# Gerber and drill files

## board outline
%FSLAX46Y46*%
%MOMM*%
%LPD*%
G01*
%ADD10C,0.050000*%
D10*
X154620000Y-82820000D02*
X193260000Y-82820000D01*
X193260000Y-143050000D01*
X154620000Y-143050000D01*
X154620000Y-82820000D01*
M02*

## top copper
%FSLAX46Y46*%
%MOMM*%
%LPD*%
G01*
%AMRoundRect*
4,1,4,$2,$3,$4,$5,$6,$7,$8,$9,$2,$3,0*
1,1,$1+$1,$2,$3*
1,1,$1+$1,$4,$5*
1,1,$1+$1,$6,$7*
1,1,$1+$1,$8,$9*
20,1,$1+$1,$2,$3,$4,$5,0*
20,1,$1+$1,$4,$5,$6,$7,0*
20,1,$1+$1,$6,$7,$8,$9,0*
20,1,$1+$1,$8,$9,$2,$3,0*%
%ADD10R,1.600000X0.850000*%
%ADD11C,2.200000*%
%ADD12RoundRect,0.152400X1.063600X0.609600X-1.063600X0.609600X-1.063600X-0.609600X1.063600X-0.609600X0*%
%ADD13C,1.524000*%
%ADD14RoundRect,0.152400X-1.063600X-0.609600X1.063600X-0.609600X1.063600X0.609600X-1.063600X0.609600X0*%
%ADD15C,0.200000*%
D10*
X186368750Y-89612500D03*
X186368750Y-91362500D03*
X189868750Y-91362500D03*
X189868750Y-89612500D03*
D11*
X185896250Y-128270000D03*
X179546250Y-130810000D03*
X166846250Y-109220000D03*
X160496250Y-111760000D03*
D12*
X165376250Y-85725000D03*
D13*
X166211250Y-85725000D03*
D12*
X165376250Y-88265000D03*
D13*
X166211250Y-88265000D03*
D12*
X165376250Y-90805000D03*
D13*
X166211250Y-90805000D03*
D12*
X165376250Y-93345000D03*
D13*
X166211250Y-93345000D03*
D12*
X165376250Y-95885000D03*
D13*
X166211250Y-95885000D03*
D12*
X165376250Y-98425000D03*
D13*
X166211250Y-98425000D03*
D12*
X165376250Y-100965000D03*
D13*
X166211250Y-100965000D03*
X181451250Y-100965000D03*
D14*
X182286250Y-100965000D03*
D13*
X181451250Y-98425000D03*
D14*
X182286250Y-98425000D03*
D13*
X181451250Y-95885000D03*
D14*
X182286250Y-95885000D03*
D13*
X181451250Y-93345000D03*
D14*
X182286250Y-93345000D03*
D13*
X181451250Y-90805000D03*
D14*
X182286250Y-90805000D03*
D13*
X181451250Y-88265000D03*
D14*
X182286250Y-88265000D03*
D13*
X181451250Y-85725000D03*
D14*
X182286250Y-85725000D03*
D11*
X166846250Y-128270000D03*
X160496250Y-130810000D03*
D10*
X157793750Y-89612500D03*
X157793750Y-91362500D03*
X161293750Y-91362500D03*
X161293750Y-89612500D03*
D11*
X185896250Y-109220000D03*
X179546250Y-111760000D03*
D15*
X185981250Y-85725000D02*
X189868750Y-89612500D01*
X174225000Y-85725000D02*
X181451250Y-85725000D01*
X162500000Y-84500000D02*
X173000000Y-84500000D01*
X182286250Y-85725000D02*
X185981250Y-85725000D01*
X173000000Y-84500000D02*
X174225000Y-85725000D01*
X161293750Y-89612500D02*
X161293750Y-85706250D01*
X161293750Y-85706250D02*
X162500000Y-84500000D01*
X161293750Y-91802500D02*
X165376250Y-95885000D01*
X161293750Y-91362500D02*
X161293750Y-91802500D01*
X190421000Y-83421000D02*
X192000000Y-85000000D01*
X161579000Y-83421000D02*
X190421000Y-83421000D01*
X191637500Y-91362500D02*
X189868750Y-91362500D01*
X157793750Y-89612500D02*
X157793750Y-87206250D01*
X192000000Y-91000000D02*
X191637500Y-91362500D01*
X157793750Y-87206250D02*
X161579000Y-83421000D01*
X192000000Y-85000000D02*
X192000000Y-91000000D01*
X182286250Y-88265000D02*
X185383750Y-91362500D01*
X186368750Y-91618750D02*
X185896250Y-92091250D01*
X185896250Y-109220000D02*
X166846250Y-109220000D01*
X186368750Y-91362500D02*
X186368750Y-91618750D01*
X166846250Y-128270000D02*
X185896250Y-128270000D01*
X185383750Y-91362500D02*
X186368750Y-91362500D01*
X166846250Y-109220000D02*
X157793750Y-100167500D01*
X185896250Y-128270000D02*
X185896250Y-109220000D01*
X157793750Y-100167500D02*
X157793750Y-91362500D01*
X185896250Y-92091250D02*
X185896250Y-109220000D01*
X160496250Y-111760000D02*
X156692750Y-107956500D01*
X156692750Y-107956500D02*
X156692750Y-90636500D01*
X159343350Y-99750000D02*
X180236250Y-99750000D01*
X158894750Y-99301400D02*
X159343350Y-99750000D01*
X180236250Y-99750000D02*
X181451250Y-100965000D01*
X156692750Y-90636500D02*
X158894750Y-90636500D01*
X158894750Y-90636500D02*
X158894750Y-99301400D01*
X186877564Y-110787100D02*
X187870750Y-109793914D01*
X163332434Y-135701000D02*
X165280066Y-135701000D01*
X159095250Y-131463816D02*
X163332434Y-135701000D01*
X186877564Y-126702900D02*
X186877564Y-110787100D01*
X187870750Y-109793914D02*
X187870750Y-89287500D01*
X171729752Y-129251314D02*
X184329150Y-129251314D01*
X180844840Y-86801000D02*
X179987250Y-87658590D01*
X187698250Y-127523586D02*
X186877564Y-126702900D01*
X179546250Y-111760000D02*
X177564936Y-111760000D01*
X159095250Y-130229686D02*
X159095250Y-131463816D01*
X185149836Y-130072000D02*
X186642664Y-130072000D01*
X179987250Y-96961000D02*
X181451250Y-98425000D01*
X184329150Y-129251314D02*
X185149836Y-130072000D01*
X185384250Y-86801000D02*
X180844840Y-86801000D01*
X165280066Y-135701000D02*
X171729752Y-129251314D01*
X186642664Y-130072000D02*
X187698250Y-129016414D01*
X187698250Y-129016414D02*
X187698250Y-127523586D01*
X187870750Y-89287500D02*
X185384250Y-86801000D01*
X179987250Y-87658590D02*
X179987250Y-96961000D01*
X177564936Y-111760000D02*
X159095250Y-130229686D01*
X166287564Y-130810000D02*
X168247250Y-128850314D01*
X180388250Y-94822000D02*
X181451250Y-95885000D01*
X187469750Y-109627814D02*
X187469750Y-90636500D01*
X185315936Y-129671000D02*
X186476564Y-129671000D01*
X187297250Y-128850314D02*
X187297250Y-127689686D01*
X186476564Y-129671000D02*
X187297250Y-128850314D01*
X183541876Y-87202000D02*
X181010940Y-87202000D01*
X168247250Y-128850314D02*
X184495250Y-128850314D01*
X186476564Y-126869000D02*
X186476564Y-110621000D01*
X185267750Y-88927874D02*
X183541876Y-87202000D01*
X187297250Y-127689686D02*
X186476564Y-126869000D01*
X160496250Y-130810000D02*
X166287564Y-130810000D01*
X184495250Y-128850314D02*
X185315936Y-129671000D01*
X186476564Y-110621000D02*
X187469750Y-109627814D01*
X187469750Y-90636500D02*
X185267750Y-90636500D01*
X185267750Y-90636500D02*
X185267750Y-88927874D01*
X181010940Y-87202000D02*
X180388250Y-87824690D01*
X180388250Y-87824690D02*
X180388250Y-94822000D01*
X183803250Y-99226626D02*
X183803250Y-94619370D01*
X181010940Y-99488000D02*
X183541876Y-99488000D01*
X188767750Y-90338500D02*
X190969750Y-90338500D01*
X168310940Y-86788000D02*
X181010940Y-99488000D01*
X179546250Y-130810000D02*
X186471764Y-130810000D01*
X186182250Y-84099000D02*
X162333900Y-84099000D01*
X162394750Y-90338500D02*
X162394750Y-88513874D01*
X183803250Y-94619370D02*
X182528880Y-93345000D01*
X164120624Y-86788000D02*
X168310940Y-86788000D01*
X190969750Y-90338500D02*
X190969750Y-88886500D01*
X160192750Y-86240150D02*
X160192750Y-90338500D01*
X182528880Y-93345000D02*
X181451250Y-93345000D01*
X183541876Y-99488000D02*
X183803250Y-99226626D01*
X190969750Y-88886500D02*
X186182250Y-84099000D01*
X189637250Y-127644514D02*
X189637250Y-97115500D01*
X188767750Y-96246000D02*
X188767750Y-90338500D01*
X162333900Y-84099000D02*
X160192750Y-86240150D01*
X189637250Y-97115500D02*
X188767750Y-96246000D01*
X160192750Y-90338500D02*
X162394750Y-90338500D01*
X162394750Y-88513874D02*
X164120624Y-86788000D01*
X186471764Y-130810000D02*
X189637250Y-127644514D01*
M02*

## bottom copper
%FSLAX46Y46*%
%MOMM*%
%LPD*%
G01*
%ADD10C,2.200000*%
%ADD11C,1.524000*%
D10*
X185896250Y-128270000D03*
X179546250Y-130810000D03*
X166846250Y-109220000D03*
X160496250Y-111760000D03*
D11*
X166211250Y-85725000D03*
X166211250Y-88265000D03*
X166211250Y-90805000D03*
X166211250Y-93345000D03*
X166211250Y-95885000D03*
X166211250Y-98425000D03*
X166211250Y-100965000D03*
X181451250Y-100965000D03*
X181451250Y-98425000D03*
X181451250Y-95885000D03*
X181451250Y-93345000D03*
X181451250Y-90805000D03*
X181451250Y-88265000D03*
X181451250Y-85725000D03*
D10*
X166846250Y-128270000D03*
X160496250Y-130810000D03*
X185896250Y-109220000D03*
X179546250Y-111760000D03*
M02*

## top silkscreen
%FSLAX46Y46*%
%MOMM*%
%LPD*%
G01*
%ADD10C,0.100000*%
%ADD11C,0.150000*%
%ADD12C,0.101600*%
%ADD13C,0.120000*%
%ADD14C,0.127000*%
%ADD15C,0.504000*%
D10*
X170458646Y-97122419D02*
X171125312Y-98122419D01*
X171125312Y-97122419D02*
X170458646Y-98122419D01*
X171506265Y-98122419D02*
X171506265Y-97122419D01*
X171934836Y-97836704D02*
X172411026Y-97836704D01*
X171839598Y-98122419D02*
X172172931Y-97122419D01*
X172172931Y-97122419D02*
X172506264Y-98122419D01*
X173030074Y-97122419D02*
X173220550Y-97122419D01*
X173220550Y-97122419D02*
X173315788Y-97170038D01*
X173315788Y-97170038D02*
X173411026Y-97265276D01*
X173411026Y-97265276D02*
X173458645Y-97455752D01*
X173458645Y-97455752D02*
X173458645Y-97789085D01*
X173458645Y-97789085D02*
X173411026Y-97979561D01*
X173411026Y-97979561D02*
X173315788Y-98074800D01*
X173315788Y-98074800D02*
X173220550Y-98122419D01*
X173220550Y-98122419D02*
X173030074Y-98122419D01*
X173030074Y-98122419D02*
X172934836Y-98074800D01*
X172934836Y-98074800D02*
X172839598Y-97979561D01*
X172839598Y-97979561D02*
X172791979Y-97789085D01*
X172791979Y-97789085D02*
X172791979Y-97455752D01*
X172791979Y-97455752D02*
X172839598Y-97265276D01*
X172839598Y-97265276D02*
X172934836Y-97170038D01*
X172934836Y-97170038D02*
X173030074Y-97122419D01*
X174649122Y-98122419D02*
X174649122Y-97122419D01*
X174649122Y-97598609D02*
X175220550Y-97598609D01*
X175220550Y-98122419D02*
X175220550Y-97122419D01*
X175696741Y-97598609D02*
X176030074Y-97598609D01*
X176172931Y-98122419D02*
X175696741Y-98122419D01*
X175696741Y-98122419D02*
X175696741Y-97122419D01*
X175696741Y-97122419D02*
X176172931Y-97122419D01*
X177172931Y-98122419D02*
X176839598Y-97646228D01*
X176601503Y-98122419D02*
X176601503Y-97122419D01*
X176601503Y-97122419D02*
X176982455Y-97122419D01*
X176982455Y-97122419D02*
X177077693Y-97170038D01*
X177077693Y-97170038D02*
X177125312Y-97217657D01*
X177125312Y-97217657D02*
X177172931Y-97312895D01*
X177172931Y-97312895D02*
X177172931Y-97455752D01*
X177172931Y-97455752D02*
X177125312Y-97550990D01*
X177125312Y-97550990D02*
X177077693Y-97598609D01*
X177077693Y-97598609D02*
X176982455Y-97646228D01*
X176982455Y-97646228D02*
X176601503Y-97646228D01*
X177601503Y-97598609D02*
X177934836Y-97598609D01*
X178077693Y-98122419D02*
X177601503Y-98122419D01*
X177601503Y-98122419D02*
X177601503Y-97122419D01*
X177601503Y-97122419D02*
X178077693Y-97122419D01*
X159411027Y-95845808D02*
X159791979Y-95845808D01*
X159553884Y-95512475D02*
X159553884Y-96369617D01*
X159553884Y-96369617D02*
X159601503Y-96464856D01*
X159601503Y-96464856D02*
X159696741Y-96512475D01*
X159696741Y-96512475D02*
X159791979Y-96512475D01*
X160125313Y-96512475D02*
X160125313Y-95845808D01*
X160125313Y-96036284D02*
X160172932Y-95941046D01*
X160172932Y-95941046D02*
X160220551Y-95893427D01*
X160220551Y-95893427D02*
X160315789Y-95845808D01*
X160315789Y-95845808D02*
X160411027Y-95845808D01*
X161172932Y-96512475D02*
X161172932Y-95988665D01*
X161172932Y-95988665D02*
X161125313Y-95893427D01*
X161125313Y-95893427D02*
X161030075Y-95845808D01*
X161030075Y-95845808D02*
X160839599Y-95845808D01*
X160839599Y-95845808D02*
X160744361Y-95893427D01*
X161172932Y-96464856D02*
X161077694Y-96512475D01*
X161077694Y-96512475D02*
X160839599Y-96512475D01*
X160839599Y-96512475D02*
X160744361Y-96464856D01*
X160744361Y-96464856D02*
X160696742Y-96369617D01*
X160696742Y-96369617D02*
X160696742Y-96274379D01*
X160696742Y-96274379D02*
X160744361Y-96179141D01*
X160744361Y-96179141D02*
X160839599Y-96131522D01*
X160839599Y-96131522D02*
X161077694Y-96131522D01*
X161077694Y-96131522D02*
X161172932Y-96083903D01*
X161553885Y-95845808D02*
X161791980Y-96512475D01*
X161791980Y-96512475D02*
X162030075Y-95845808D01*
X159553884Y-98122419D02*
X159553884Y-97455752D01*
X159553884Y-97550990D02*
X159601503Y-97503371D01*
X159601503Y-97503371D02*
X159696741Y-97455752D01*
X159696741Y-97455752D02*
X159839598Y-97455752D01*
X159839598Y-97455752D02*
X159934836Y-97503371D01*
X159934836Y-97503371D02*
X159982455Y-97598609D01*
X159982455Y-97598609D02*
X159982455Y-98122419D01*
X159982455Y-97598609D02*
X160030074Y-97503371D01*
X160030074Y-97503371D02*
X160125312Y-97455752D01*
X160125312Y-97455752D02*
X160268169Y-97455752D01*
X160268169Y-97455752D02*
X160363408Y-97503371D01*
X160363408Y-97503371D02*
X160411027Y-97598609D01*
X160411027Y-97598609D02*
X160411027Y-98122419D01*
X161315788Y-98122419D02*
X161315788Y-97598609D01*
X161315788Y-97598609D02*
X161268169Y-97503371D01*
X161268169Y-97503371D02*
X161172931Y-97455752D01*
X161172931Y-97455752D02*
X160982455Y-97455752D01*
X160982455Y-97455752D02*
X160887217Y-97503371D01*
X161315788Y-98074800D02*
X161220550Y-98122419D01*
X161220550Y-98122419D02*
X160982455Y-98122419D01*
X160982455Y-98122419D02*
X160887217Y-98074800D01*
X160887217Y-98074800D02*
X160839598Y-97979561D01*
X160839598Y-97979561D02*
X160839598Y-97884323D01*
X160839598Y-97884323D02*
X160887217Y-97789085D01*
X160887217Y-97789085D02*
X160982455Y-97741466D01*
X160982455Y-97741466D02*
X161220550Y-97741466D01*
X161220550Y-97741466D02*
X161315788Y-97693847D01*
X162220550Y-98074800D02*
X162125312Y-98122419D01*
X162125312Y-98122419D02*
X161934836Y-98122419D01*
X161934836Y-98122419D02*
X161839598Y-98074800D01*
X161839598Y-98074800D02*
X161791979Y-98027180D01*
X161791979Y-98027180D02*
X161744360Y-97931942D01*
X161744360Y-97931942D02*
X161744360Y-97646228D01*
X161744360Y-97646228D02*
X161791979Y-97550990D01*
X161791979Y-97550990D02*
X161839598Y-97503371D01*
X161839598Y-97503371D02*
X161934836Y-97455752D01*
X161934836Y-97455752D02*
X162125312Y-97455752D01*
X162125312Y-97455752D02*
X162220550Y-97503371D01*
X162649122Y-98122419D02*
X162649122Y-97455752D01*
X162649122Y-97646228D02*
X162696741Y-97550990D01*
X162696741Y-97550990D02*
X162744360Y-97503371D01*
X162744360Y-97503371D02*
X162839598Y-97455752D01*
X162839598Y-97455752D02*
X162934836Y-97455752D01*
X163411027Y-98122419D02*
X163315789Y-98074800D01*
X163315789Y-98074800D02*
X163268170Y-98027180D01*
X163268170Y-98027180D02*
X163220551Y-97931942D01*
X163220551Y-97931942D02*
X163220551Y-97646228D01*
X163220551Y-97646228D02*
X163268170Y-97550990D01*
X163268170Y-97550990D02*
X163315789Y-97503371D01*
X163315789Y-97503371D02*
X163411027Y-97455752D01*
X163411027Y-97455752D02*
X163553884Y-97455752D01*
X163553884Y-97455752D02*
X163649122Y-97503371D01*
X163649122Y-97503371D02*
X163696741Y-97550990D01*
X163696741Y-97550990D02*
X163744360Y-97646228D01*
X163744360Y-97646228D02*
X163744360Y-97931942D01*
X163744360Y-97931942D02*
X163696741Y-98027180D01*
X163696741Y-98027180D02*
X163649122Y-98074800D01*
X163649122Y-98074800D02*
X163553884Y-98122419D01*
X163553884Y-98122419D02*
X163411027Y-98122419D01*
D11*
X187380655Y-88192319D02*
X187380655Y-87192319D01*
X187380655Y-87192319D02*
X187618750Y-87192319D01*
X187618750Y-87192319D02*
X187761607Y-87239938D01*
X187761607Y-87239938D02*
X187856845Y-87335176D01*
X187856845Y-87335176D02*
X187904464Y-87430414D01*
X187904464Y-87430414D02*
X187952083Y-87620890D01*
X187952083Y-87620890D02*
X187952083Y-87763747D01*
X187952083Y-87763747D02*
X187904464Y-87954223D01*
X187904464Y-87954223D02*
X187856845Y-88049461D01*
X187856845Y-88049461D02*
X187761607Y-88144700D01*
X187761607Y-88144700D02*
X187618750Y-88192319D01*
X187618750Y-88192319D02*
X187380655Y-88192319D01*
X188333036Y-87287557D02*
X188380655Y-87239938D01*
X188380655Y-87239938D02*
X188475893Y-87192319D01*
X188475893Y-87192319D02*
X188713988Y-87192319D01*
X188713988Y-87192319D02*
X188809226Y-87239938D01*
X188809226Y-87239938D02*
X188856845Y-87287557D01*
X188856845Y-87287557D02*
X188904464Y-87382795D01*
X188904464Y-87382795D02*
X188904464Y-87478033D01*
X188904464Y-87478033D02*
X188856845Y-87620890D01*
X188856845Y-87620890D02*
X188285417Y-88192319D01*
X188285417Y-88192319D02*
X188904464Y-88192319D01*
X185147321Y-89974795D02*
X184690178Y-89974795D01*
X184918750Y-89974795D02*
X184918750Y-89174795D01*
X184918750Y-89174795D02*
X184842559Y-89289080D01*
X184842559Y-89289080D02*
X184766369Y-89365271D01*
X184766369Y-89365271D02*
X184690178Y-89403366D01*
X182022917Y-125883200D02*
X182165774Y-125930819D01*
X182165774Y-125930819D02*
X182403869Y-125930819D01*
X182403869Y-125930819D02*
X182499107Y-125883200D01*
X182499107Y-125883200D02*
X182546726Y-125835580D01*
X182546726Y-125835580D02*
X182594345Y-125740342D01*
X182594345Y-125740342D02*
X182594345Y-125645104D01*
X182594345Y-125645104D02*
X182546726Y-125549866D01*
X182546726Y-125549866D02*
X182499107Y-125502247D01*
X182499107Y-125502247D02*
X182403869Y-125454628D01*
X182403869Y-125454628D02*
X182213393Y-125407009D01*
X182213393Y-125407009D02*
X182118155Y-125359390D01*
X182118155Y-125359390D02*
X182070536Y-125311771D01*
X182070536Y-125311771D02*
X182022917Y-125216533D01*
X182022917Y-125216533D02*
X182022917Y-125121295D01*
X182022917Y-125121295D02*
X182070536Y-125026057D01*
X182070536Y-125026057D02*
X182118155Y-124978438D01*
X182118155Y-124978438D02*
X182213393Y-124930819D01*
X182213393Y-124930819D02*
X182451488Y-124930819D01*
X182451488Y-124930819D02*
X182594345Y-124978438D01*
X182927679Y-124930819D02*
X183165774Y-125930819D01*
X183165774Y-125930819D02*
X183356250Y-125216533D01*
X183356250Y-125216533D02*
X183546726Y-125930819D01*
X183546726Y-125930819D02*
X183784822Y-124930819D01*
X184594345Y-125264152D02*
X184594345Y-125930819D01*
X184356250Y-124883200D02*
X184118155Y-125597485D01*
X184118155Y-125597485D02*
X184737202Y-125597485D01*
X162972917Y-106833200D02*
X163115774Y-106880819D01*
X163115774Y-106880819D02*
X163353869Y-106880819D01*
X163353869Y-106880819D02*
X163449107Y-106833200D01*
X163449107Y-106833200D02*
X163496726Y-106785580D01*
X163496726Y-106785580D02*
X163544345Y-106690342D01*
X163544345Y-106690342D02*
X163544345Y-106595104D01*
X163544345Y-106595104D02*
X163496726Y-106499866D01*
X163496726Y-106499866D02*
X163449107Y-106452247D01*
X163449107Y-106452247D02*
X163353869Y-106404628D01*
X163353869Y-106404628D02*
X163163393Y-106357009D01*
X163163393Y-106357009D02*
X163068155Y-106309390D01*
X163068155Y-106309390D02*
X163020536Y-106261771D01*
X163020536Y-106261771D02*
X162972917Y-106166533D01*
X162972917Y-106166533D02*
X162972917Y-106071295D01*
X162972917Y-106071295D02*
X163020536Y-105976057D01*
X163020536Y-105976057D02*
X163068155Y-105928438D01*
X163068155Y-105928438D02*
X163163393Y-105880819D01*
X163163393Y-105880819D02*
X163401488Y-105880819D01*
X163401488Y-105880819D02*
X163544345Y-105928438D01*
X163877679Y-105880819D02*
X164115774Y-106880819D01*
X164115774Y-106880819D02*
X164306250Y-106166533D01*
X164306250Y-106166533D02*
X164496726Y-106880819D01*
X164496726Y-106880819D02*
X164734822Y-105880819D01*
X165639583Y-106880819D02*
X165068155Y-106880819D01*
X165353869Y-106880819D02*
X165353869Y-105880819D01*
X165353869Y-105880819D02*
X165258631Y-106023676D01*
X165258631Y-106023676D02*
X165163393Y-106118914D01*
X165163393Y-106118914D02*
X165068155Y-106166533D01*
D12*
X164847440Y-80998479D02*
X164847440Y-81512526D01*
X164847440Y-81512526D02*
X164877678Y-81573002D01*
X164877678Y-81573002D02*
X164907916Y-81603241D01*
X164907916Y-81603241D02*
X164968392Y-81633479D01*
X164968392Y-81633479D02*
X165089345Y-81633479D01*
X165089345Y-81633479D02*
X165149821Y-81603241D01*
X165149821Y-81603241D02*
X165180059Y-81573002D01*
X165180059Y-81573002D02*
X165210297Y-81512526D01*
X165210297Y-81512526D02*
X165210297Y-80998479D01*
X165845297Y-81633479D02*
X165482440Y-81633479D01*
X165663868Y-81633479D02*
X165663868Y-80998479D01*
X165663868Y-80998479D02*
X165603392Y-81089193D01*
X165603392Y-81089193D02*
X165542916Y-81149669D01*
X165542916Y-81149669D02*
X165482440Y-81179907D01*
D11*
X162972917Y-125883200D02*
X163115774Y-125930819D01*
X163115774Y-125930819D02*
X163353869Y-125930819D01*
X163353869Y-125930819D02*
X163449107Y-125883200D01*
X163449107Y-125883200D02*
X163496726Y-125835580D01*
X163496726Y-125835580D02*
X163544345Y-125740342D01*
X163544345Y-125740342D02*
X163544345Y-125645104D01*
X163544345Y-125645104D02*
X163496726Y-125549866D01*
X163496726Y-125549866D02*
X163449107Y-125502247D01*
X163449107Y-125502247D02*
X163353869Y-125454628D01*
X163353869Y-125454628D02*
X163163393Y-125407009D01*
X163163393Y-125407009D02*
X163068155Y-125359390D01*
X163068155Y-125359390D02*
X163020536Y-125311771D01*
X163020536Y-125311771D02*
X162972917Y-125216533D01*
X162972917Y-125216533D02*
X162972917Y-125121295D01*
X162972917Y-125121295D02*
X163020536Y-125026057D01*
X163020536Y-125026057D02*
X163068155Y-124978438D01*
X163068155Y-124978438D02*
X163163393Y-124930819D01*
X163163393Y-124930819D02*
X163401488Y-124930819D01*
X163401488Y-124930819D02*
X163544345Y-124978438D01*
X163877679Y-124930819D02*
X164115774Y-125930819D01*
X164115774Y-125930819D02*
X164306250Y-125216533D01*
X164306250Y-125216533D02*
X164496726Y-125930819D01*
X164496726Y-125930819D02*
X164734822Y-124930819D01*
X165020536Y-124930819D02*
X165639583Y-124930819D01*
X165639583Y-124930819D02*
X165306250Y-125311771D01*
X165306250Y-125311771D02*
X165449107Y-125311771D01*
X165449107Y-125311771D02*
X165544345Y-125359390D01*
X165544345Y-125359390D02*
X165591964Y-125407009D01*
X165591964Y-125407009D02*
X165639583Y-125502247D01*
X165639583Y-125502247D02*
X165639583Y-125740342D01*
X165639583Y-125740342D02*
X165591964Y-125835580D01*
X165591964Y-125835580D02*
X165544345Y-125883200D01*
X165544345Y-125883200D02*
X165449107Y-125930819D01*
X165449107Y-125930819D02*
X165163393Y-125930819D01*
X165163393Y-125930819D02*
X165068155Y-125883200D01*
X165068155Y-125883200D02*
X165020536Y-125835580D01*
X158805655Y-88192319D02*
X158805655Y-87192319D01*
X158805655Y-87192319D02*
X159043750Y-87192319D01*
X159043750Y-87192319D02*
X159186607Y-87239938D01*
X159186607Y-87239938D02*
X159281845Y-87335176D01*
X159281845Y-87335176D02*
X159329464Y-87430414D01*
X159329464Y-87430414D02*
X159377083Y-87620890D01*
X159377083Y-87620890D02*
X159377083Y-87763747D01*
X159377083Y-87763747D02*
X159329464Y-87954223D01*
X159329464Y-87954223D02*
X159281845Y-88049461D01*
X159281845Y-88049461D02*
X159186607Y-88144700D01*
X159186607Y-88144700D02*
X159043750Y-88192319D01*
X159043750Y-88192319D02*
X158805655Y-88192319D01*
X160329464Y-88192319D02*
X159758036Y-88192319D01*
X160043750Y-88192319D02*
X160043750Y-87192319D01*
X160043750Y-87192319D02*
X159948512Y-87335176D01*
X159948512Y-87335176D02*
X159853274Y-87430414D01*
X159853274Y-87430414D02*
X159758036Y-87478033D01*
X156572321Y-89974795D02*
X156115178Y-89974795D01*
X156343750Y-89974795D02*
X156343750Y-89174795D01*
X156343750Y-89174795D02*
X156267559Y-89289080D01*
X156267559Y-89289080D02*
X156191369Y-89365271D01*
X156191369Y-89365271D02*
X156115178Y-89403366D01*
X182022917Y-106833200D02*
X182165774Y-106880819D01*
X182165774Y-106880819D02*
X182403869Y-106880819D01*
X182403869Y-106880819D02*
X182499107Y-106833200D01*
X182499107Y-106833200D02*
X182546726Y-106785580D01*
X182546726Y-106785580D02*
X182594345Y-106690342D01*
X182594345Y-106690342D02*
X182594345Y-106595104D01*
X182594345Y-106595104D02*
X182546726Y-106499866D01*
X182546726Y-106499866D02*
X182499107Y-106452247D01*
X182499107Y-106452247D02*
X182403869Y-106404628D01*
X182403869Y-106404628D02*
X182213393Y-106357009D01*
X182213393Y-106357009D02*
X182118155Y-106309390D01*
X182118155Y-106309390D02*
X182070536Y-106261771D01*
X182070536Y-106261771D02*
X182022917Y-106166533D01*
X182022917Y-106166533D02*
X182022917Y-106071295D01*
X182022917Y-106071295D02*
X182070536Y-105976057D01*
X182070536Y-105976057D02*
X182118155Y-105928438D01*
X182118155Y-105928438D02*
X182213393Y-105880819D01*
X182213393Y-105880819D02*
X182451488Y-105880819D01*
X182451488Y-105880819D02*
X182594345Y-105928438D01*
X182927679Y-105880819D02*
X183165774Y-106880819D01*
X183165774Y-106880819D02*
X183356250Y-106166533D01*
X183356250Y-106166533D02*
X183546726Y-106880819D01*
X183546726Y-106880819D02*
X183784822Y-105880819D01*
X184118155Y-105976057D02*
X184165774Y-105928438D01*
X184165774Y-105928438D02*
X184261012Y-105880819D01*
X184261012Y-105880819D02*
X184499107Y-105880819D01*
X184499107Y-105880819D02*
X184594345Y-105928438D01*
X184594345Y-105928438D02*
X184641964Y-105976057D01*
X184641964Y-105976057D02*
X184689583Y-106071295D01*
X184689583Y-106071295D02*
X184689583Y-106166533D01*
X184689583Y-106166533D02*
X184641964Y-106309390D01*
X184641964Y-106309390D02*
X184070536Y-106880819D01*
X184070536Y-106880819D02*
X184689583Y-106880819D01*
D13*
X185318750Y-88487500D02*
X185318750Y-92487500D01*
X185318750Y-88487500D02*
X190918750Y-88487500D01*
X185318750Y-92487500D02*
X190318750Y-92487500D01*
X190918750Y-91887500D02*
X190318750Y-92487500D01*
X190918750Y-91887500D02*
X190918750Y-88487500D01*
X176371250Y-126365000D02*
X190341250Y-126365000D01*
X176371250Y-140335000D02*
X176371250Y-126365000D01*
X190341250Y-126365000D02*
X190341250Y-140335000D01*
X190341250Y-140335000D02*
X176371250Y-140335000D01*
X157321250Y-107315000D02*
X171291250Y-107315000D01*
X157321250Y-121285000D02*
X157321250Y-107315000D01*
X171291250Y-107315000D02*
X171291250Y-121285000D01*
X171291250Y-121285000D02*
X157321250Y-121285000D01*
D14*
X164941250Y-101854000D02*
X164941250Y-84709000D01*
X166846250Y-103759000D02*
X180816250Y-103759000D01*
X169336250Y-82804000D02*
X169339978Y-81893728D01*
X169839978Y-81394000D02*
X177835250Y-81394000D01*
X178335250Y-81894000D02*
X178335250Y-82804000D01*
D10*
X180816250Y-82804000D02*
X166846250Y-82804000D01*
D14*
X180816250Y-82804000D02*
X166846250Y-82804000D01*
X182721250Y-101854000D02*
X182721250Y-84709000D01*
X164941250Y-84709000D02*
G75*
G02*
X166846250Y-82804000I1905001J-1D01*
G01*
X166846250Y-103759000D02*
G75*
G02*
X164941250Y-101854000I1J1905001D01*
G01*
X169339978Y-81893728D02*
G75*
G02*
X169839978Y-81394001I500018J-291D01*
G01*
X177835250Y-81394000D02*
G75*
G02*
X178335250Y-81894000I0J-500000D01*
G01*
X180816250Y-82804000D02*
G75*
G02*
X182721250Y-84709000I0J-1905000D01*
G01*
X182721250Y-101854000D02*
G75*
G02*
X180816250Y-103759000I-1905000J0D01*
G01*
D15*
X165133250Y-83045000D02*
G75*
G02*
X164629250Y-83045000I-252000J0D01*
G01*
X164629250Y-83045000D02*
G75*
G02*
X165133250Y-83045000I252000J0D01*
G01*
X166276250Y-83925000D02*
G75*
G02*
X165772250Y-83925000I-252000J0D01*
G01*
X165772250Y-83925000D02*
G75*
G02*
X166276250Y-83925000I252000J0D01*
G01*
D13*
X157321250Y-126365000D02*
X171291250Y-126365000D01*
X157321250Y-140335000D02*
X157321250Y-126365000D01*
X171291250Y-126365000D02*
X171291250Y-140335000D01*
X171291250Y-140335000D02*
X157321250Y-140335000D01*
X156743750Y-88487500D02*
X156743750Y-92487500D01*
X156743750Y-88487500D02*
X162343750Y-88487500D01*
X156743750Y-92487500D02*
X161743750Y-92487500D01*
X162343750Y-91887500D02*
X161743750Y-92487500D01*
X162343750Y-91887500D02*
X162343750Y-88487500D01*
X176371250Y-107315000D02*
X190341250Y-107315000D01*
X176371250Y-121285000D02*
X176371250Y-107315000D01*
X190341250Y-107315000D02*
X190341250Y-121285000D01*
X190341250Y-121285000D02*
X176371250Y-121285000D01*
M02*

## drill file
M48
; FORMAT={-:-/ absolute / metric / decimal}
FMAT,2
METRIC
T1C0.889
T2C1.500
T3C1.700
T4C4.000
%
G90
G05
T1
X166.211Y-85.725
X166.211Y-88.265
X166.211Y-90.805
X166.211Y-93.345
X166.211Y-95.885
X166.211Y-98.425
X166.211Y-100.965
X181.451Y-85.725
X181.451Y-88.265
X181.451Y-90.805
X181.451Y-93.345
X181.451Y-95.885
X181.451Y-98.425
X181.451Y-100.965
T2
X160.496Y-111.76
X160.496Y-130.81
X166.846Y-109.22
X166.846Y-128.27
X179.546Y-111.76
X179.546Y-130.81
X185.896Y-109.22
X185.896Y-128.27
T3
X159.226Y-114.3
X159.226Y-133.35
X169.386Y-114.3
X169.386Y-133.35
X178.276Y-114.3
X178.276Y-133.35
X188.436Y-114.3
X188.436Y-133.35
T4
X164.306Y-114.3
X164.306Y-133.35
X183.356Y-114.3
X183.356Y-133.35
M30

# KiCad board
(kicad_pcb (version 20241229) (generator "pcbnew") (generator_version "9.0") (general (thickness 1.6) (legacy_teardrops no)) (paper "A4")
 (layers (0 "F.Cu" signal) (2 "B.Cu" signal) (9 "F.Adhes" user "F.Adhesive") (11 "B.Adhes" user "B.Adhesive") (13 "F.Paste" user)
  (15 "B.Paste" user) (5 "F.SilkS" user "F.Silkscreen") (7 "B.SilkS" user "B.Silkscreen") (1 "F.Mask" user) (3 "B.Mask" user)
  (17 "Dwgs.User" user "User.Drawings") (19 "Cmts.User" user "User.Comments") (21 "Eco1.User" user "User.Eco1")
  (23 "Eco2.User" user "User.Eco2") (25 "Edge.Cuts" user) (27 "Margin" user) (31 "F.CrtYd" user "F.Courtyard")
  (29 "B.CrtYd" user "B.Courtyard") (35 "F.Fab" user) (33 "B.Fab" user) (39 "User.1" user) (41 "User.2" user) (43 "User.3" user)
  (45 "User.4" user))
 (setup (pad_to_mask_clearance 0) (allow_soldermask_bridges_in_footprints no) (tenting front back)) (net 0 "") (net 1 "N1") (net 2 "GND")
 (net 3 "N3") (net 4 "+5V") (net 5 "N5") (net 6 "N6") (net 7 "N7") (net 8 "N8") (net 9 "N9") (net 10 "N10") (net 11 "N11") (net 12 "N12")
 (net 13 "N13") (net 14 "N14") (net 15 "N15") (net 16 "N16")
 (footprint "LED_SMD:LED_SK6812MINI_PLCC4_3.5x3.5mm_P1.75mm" (layer "F.Cu") (at 188.11875 90.4875)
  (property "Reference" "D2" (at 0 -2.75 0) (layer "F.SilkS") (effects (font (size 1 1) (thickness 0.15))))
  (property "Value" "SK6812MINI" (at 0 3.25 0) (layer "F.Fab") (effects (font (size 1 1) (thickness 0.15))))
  (fp_line (start -2.8 -2) (end -2.8 2) (stroke (width 0.12) (type default)) (layer "F.SilkS"))
  (fp_line (start -2.8 -2) (end 2.8 -2) (stroke (width 0.12) (type solid)) (layer "F.SilkS"))
  (fp_line (start -2.8 2) (end 2.2 2) (stroke (width 0.12) (type solid)) (layer "F.SilkS"))
  (fp_line (start 2.8 1.4) (end 2.2 2) (stroke (width 0.12) (type default)) (layer "F.SilkS"))
  (fp_line (start 2.8 1.4) (end 2.8 -2) (stroke (width 0.12) (type solid)) (layer "F.SilkS"))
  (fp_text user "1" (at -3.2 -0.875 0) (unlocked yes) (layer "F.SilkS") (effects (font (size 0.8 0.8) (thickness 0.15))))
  (pad "1" smd rect (at -1.75 -0.875) (size 1.6 0.85) (layers "F.Cu" "F.Mask" "F.Paste") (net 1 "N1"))
  (pad "2" smd rect (at -1.75 0.875) (size 1.6 0.85) (layers "F.Cu" "F.Mask" "F.Paste") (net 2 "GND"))
  (pad "3" smd rect (at 1.75 0.875) (size 1.6 0.85) (layers "F.Cu" "F.Mask" "F.Paste") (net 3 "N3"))
  (pad "4" smd rect (at 1.75 -0.875) (size 1.6 0.85) (layers "F.Cu" "F.Mask" "F.Paste") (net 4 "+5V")))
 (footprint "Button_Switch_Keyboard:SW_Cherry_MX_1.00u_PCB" (layer "F.Cu") (at 185.89625 128.27)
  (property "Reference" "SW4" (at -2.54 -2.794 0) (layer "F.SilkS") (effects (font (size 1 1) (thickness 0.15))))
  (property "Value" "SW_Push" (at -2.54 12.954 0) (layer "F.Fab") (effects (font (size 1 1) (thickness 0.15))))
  (fp_line (start -9.525 -1.905) (end 4.445 -1.905) (stroke (width 0.12) (type solid)) (layer "F.SilkS"))
  (fp_line (start -9.525 12.065) (end -9.525 -1.905) (stroke (width 0.12) (type solid)) (layer "F.SilkS"))
  (fp_line (start 4.445 -1.905) (end 4.445 12.065) (stroke (width 0.12) (type solid)) (layer "F.SilkS"))
  (fp_line (start 4.445 12.065) (end -9.525 12.065) (stroke (width 0.12) (type solid)) (layer "F.SilkS"))
  (pad "" np_thru_hole circle (at -7.62 5.08) (size 1.7 1.7) (drill 1.7) (layers "*.Cu" "*.Mask"))
  (pad "" np_thru_hole circle (at -2.54 5.08) (size 4 4) (drill 4) (layers "*.Cu" "*.Mask"))
  (pad "" np_thru_hole circle (at 2.54 5.08) (size 1.7 1.7) (drill 1.7) (layers "*.Cu" "*.Mask"))
  (pad "1" thru_hole circle (at 0 0) (size 2.2 2.2) (drill 1.5) (layers "*.Cu" "*.Mask") (remove_unused_layers no) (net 2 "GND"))
  (pad "2" thru_hole circle (at -6.35 2.54) (size 2.2 2.2) (drill 1.5) (layers "*.Cu" "*.Mask") (remove_unused_layers no) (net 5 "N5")))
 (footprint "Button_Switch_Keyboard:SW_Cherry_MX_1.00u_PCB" (layer "F.Cu") (at 166.84625 109.22)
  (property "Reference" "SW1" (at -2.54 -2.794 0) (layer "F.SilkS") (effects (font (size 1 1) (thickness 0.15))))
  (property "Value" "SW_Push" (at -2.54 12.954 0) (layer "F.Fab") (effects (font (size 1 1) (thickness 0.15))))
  (fp_line (start -9.525 -1.905) (end 4.445 -1.905) (stroke (width 0.12) (type solid)) (layer "F.SilkS"))
  (fp_line (start -9.525 12.065) (end -9.525 -1.905) (stroke (width 0.12) (type solid)) (layer "F.SilkS"))
  (fp_line (start 4.445 -1.905) (end 4.445 12.065) (stroke (width 0.12) (type solid)) (layer "F.SilkS"))
  (fp_line (start 4.445 12.065) (end -9.525 12.065) (stroke (width 0.12) (type solid)) (layer "F.SilkS"))
  (pad "" np_thru_hole circle (at -7.62 5.08) (size 1.7 1.7) (drill 1.7) (layers "*.Cu" "*.Mask"))
  (pad "" np_thru_hole circle (at -2.54 5.08) (size 4 4) (drill 4) (layers "*.Cu" "*.Mask"))
  (pad "" np_thru_hole circle (at 2.54 5.08) (size 1.7 1.7) (drill 1.7) (layers "*.Cu" "*.Mask"))
  (pad "1" thru_hole circle (at 0 0) (size 2.2 2.2) (drill 1.5) (layers "*.Cu" "*.Mask") (remove_unused_layers no) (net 2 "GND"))
  (pad "2" thru_hole circle (at -6.35 2.54) (size 2.2 2.2) (drill 1.5) (layers "*.Cu" "*.Mask") (remove_unused_layers no) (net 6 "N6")))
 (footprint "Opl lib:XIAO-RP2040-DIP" (layer "F.Cu") (at 173.83125 93.345)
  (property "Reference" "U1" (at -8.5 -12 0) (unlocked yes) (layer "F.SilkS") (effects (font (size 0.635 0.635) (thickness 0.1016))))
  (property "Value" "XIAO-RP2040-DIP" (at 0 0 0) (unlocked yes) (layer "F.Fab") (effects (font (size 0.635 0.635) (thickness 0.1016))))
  (fp_line (start -8.89 8.509) (end -8.89 -8.636) (stroke (width 0.127) (type solid)) (layer "F.SilkS"))
  (fp_line (start -6.985 10.414) (end 6.985 10.414) (stroke (width 0.127) (type solid)) (layer "F.SilkS"))
  (fp_line (start -4.495 -10.541) (end -4.491272 -11.451272) (stroke (width 0.127) (type solid)) (layer "F.SilkS"))
  (fp_line (start -3.991272 -11.951) (end 4.004 -11.951) (stroke (width 0.127) (type solid)) (layer "F.SilkS"))
  (fp_line (start 4.504 -11.451) (end 4.504 -10.541) (stroke (width 0.127) (type solid)) (layer "F.SilkS"))
  (fp_line (start 6.985 -10.541) (end -6.985 -10.541) (stroke (width 0.1) (type solid)) (layer "F.SilkS"))
  (fp_line (start 6.985 -10.541) (end -6.985 -10.541) (stroke (width 0.127) (type solid)) (layer "F.SilkS"))
  (fp_line (start 8.89 8.509) (end 8.89 -8.636) (stroke (width 0.127) (type solid)) (layer "F.SilkS"))
  (fp_arc (start -8.89 -8.636) (mid -8.332038 -9.983038) (end -6.985 -10.541) (stroke (width 0.127) (type solid)) (layer "F.SilkS"))
  (fp_arc (start -6.985 10.414) (mid -8.332038 9.856038) (end -8.89 8.509) (stroke (width 0.127) (type solid)) (layer "F.SilkS"))
  (fp_arc (start -4.491272 -11.451272) (mid -4.344728 -11.80464) (end -3.991272 -11.951) (stroke (width 0.127) (type default))
   (layer "F.SilkS"))
  (fp_arc (start 4.004 -11.951) (mid 4.357553 -11.804553) (end 4.504 -11.451) (stroke (width 0.127) (type default)) (layer "F.SilkS"))
  (fp_arc (start 6.985 -10.541) (mid 8.332038 -9.983038) (end 8.89 -8.636) (stroke (width 0.127) (type solid)) (layer "F.SilkS"))
  (fp_arc (start 8.89 8.509) (mid 8.332038 9.856038) (end 6.985 10.414) (stroke (width 0.127) (type solid)) (layer "F.SilkS"))
  (fp_circle (center -8.95 -10.3) (end -8.95 -10.554) (stroke (width 0.5) (type solid)) (fill yes) (layer "F.SilkS"))
  (fp_circle (center -7.807 -9.42) (end -7.807 -9.674) (stroke (width 0.5) (type solid)) (fill yes) (layer "F.SilkS"))
  (pad "1" smd roundrect (at -8.455 -7.62 180) (size 2.432 1.524) (layers "F.Cu" "F.Mask") (roundrect_rratio 0.1) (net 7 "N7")
   (thermal_bridge_angle 45))
  (pad "1" thru_hole circle (at -7.62 -7.62 180) (size 1.524 1.524) (drill 0.889) (layers "*.Cu" "*.Mask") (remove_unused_layers no)
   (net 7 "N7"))
  (pad "2" smd roundrect (at -8.455 -5.08 180) (size 2.432 1.524) (layers "F.Cu" "F.Mask") (roundrect_rratio 0.1) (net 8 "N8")
   (thermal_bridge_angle 45))
  (pad "2" thru_hole circle (at -7.62 -5.08 180) (size 1.524 1.524) (drill 0.889) (layers "*.Cu" "*.Mask") (remove_unused_layers no)
   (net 8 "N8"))
  (pad "3" smd roundrect (at -8.455 -2.54 180) (size 2.432 1.524) (layers "F.Cu" "F.Mask") (roundrect_rratio 0.1) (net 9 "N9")
   (thermal_bridge_angle 45))
  (pad "3" thru_hole circle (at -7.62 -2.54 180) (size 1.524 1.524) (drill 0.889) (layers "*.Cu" "*.Mask") (remove_unused_layers no)
   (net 9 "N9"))
  (pad "4" smd roundrect (at -8.455 0 180) (size 2.432 1.524) (layers "F.Cu" "F.Mask") (roundrect_rratio 0.1) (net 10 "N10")
   (thermal_bridge_angle 45))
  (pad "4" thru_hole circle (at -7.62 0 180) (size 1.524 1.524) (drill 0.889) (layers "*.Cu" "*.Mask") (remove_unused_layers no)
   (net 10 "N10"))
  (pad "5" smd roundrect (at -8.455 2.54 180) (size 2.432 1.524) (layers "F.Cu" "F.Mask") (roundrect_rratio 0.1) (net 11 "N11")
   (thermal_bridge_angle 45))
  (pad "5" thru_hole circle (at -7.62 2.54 180) (size 1.524 1.524) (drill 0.889) (layers "*.Cu" "*.Mask") (remove_unused_layers no)
   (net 11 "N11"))
  (pad "6" smd roundrect (at -8.455 5.08 180) (size 2.432 1.524) (layers "F.Cu" "F.Mask") (roundrect_rratio 0.1) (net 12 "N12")
   (thermal_bridge_angle 45))
  (pad "6" thru_hole circle (at -7.62 5.08 180) (size 1.524 1.524) (drill 0.889) (layers "*.Cu" "*.Mask") (remove_unused_layers no)
   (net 12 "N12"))
  (pad "7" smd roundrect (at -8.455 7.62 180) (size 2.432 1.524) (layers "F.Cu" "F.Mask") (roundrect_rratio 0.1) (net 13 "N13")
   (thermal_bridge_angle 45))
  (pad "7" thru_hole circle (at -7.62 7.62 180) (size 1.524 1.524) (drill 0.889) (layers "*.Cu" "*.Mask") (remove_unused_layers no)
   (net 13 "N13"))
  (pad "8" thru_hole circle (at 7.62 7.62) (size 1.524 1.524) (drill 0.889) (layers "*.Cu" "*.Mask") (remove_unused_layers no) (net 6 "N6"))
  (pad "8" smd roundrect (at 8.455 7.62) (size 2.432 1.524) (layers "F.Cu" "F.Mask") (roundrect_rratio 0.1) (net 6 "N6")
   (thermal_bridge_angle 45))
  (pad "9" thru_hole circle (at 7.62 5.08) (size 1.524 1.524) (drill 0.889) (layers "*.Cu" "*.Mask") (remove_unused_layers no)
   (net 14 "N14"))
  (pad "9" smd roundrect (at 8.455 5.08) (size 2.432 1.524) (layers "F.Cu" "F.Mask") (roundrect_rratio 0.1) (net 14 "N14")
   (thermal_bridge_angle 45))
  (pad "10" thru_hole circle (at 7.62 2.54) (size 1.524 1.524) (drill 0.889) (layers "*.Cu" "*.Mask") (remove_unused_layers no)
   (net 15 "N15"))
  (pad "10" smd roundrect (at 8.455 2.54) (size 2.432 1.524) (layers "F.Cu" "F.Mask") (roundrect_rratio 0.1) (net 15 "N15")
   (thermal_bridge_angle 45))
  (pad "11" thru_hole circle (at 7.62 0) (size 1.524 1.524) (drill 0.889) (layers "*.Cu" "*.Mask") (remove_unused_layers no) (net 5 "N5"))
  (pad "11" smd roundrect (at 8.455 0) (size 2.432 1.524) (layers "F.Cu" "F.Mask") (roundrect_rratio 0.1) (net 5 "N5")
   (thermal_bridge_angle 45))
  (pad "12" thru_hole circle (at 7.62 -2.54) (size 1.524 1.524) (drill 0.889) (layers "*.Cu" "*.Mask") (remove_unused_layers no)
   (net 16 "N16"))
  (pad "12" smd roundrect (at 8.455 -2.54) (size 2.432 1.524) (layers "F.Cu" "F.Mask") (roundrect_rratio 0.1) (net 16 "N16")
   (thermal_bridge_angle 45))
  (pad "13" thru_hole circle (at 7.62 -5.08) (size 1.524 1.524) (drill 0.889) (layers "*.Cu" "*.Mask") (remove_unused_layers no)
   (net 2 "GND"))
  (pad "13" smd roundrect (at 8.455 -5.08) (size 2.432 1.524) (layers "F.Cu" "F.Mask") (roundrect_rratio 0.1) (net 2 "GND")
   (thermal_bridge_angle 45))
  (pad "14" thru_hole circle (at 7.62 -7.62) (size 1.524 1.524) (drill 0.889) (layers "*.Cu" "*.Mask") (remove_unused_layers no)
   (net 4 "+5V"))
  (pad "14" smd roundrect (at 8.455 -7.62) (size 2.432 1.524) (layers "F.Cu" "F.Mask") (roundrect_rratio 0.1) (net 4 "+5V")
   (thermal_bridge_angle 45)))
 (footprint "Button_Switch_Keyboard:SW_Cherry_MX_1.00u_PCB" (layer "F.Cu") (at 166.84625 128.27)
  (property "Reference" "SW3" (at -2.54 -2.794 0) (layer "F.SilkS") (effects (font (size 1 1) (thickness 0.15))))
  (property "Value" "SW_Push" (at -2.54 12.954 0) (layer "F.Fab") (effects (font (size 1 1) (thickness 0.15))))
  (fp_line (start -9.525 -1.905) (end 4.445 -1.905) (stroke (width 0.12) (type solid)) (layer "F.SilkS"))
  (fp_line (start -9.525 12.065) (end -9.525 -1.905) (stroke (width 0.12) (type solid)) (layer "F.SilkS"))
  (fp_line (start 4.445 -1.905) (end 4.445 12.065) (stroke (width 0.12) (type solid)) (layer "F.SilkS"))
  (fp_line (start 4.445 12.065) (end -9.525 12.065) (stroke (width 0.12) (type solid)) (layer "F.SilkS"))
  (pad "" np_thru_hole circle (at -7.62 5.08) (size 1.7 1.7) (drill 1.7) (layers "*.Cu" "*.Mask"))
  (pad "" np_thru_hole circle (at -2.54 5.08) (size 4 4) (drill 4) (layers "*.Cu" "*.Mask"))
  (pad "" np_thru_hole circle (at 2.54 5.08) (size 1.7 1.7) (drill 1.7) (layers "*.Cu" "*.Mask"))
  (pad "1" thru_hole circle (at 0 0) (size 2.2 2.2) (drill 1.5) (layers "*.Cu" "*.Mask") (remove_unused_layers no) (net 2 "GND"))
  (pad "2" thru_hole circle (at -6.35 2.54) (size 2.2 2.2) (drill 1.5) (layers "*.Cu" "*.Mask") (remove_unused_layers no) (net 15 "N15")))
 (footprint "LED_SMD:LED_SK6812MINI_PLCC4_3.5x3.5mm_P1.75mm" (layer "F.Cu") (at 159.54375 90.4875)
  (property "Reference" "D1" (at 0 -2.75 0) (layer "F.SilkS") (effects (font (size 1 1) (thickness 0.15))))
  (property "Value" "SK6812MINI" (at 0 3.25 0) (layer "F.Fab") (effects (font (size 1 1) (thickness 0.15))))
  (fp_line (start -2.8 -2) (end -2.8 2) (stroke (width 0.12) (type default)) (layer "F.SilkS"))
  (fp_line (start -2.8 -2) (end 2.8 -2) (stroke (width 0.12) (type solid)) (layer "F.SilkS"))
  (fp_line (start -2.8 2) (end 2.2 2) (stroke (width 0.12) (type solid)) (layer "F.SilkS"))
  (fp_line (start 2.8 1.4) (end 2.2 2) (stroke (width 0.12) (type default)) (layer "F.SilkS"))
  (fp_line (start 2.8 1.4) (end 2.8 -2) (stroke (width 0.12) (type solid)) (layer "F.SilkS"))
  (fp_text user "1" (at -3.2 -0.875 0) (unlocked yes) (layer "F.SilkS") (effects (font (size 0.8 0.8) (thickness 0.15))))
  (pad "1" smd rect (at -1.75 -0.875) (size 1.6 0.85) (layers "F.Cu" "F.Mask" "F.Paste") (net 3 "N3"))
  (pad "2" smd rect (at -1.75 0.875) (size 1.6 0.85) (layers "F.Cu" "F.Mask" "F.Paste") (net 2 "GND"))
  (pad "3" smd rect (at 1.75 0.875) (size 1.6 0.85) (layers "F.Cu" "F.Mask" "F.Paste") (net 11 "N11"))
  (pad "4" smd rect (at 1.75 -0.875) (size 1.6 0.85) (layers "F.Cu" "F.Mask" "F.Paste") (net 4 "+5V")))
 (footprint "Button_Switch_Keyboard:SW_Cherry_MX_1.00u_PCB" (layer "F.Cu") (at 185.89625 109.22)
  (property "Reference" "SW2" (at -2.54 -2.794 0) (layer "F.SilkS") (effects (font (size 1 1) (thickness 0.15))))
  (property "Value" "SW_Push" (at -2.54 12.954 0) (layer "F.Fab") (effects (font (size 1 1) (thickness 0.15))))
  (fp_line (start -9.525 -1.905) (end 4.445 -1.905) (stroke (width 0.12) (type solid)) (layer "F.SilkS"))
  (fp_line (start -9.525 12.065) (end -9.525 -1.905) (stroke (width 0.12) (type solid)) (layer "F.SilkS"))
  (fp_line (start 4.445 -1.905) (end 4.445 12.065) (stroke (width 0.12) (type solid)) (layer "F.SilkS"))
  (fp_line (start 4.445 12.065) (end -9.525 12.065) (stroke (width 0.12) (type solid)) (layer "F.SilkS"))
  (pad "" np_thru_hole circle (at -7.62 5.08) (size 1.7 1.7) (drill 1.7) (layers "*.Cu" "*.Mask"))
  (pad "" np_thru_hole circle (at -2.54 5.08) (size 4 4) (drill 4) (layers "*.Cu" "*.Mask"))
  (pad "" np_thru_hole circle (at 2.54 5.08) (size 1.7 1.7) (drill 1.7) (layers "*.Cu" "*.Mask"))
  (pad "1" thru_hole circle (at 0 0) (size 2.2 2.2) (drill 1.5) (layers "*.Cu" "*.Mask") (remove_unused_layers no) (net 2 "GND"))
  (pad "2" thru_hole circle (at -6.35 2.54) (size 2.2 2.2) (drill 1.5) (layers "*.Cu" "*.Mask") (remove_unused_layers no) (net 14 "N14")))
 (gr_rect (start 154.62 82.82) (end 193.26 143.05) (stroke (width 0.05) (type default)) (fill no) (layer "Edge.Cuts"))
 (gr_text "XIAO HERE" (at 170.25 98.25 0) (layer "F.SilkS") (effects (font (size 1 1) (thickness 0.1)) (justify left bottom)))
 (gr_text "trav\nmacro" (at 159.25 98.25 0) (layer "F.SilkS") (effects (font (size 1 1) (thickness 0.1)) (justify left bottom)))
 (segment (start 185.98125 85.725) (end 189.86875 89.6125) (width 0.2) (layer "F.Cu") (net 4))
 (segment (start 174.225 85.725) (end 181.45125 85.725) (width 0.2) (layer "F.Cu") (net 4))
 (segment (start 162.5 84.5) (end 173 84.5) (width 0.2) (layer "F.Cu") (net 4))
 (segment (start 182.28625 85.725) (end 185.98125 85.725) (width 0.2) (layer "F.Cu") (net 4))
 (segment (start 173 84.5) (end 174.225 85.725) (width 0.2) (layer "F.Cu") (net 4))
 (segment (start 161.29375 89.6125) (end 161.29375 85.70625) (width 0.2) (layer "F.Cu") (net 4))
 (segment (start 161.29375 85.70625) (end 162.5 84.5) (width 0.2) (layer "F.Cu") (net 4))
 (segment (start 161.29375 91.8025) (end 165.37625 95.885) (width 0.2) (layer "F.Cu") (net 11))
 (segment (start 161.29375 91.3625) (end 161.29375 91.8025) (width 0.2) (layer "F.Cu") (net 11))
 (segment (start 190.421 83.421) (end 192 85) (width 0.2) (layer "F.Cu") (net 3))
 (segment (start 161.579 83.421) (end 190.421 83.421) (width 0.2) (layer "F.Cu") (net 3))
 (segment (start 191.6375 91.3625) (end 189.86875 91.3625) (width 0.2) (layer "F.Cu") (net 3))
 (segment (start 157.79375 89.6125) (end 157.79375 87.20625) (width 0.2) (layer "F.Cu") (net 3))
 (segment (start 192 91) (end 191.6375 91.3625) (width 0.2) (layer "F.Cu") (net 3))
 (segment (start 157.79375 87.20625) (end 161.579 83.421) (width 0.2) (layer "F.Cu") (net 3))
 (segment (start 192 85) (end 192 91) (width 0.2) (layer "F.Cu") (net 3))
 (segment (start 182.28625 88.265) (end 185.38375 91.3625) (width 0.2) (layer "F.Cu") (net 2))
 (segment (start 186.36875 91.61875) (end 185.89625 92.09125) (width 0.2) (layer "F.Cu") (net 2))
 (segment (start 185.89625 109.22) (end 166.84625 109.22) (width 0.2) (layer "F.Cu") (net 2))
 (segment (start 186.36875 91.3625) (end 186.36875 91.61875) (width 0.2) (layer "F.Cu") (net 2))
 (segment (start 166.84625 128.27) (end 185.89625 128.27) (width 0.2) (layer "F.Cu") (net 2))
 (segment (start 185.38375 91.3625) (end 186.36875 91.3625) (width 0.2) (layer "F.Cu") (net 2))
 (segment (start 166.84625 109.22) (end 157.79375 100.1675) (width 0.2) (layer "F.Cu") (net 2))
 (segment (start 185.89625 128.27) (end 185.89625 109.22) (width 0.2) (layer "F.Cu") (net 2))
 (segment (start 157.79375 100.1675) (end 157.79375 91.3625) (width 0.2) (layer "F.Cu") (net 2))
 (segment (start 185.89625 92.09125) (end 185.89625 109.22) (width 0.2) (layer "F.Cu") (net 2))
 (segment (start 160.49625 111.76) (end 156.69275 107.9565) (width 0.2) (layer "F.Cu") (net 6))
 (segment (start 156.69275 107.9565) (end 156.69275 90.6365) (width 0.2) (layer "F.Cu") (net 6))
 (segment (start 159.34335 99.75) (end 180.23625 99.75) (width 0.2) (layer "F.Cu") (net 6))
 (segment (start 158.89475 99.3014) (end 159.34335 99.75) (width 0.2) (layer "F.Cu") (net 6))
 (segment (start 180.23625 99.75) (end 181.45125 100.965) (width 0.2) (layer "F.Cu") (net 6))
 (segment (start 156.69275 90.6365) (end 158.89475 90.6365) (width 0.2) (layer "F.Cu") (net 6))
 (segment (start 158.89475 90.6365) (end 158.89475 99.3014) (width 0.2) (layer "F.Cu") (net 6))
 (segment (start 186.877564 110.7871) (end 187.87075 109.793914) (width 0.2) (layer "F.Cu") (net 14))
 (segment (start 163.332434 135.701) (end 165.280066 135.701) (width 0.2) (layer "F.Cu") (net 14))
 (segment (start 159.09525 131.463816) (end 163.332434 135.701) (width 0.2) (layer "F.Cu") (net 14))
 (segment (start 186.877564 126.7029) (end 186.877564 110.7871) (width 0.2) (layer "F.Cu") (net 14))
 (segment (start 187.87075 109.793914) (end 187.87075 89.2875) (width 0.2) (layer "F.Cu") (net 14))
 (segment (start 171.729752 129.251314) (end 184.32915 129.251314) (width 0.2) (layer "F.Cu") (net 14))
 (segment (start 180.84484 86.801) (end 179.98725 87.65859) (width 0.2) (layer "F.Cu") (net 14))
 (segment (start 187.69825 127.523586) (end 186.877564 126.7029) (width 0.2) (layer "F.Cu") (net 14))
 (segment (start 179.54625 111.76) (end 177.564936 111.76) (width 0.2) (layer "F.Cu") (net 14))
 (segment (start 159.09525 130.229686) (end 159.09525 131.463816) (width 0.2) (layer "F.Cu") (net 14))
 (segment (start 185.149836 130.072) (end 186.642664 130.072) (width 0.2) (layer "F.Cu") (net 14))
 (segment (start 179.98725 96.961) (end 181.45125 98.425) (width 0.2) (layer "F.Cu") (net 14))
 (segment (start 184.32915 129.251314) (end 185.149836 130.072) (width 0.2) (layer "F.Cu") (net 14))
 (segment (start 185.38425 86.801) (end 180.84484 86.801) (width 0.2) (layer "F.Cu") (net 14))
 (segment (start 165.280066 135.701) (end 171.729752 129.251314) (width 0.2) (layer "F.Cu") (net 14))
 (segment (start 186.642664 130.072) (end 187.69825 129.016414) (width 0.2) (layer "F.Cu") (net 14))
 (segment (start 187.69825 129.016414) (end 187.69825 127.523586) (width 0.2) (layer "F.Cu") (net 14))
 (segment (start 187.87075 89.2875) (end 185.38425 86.801) (width 0.2) (layer "F.Cu") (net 14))
 (segment (start 179.98725 87.65859) (end 179.98725 96.961) (width 0.2) (layer "F.Cu") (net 14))
 (segment (start 177.564936 111.76) (end 159.09525 130.229686) (width 0.2) (layer "F.Cu") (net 14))
 (segment (start 166.287564 130.81) (end 168.24725 128.850314) (width 0.2) (layer "F.Cu") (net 15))
 (segment (start 180.38825 94.822) (end 181.45125 95.885) (width 0.2) (layer "F.Cu") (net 15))
 (segment (start 187.46975 109.627814) (end 187.46975 90.6365) (width 0.2) (layer "F.Cu") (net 15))
 (segment (start 185.315936 129.671) (end 186.476564 129.671) (width 0.2) (layer "F.Cu") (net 15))
 (segment (start 187.29725 128.850314) (end 187.29725 127.689686) (width 0.2) (layer "F.Cu") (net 15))
 (segment (start 186.476564 129.671) (end 187.29725 128.850314) (width 0.2) (layer "F.Cu") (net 15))
 (segment (start 183.541876 87.202) (end 181.01094 87.202) (width 0.2) (layer "F.Cu") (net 15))
 (segment (start 168.24725 128.850314) (end 184.49525 128.850314) (width 0.2) (layer "F.Cu") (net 15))
 (segment (start 186.476564 126.869) (end 186.476564 110.621) (width 0.2) (layer "F.Cu") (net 15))
 (segment (start 185.26775 88.927874) (end 183.541876 87.202) (width 0.2) (layer "F.Cu") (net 15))
 (segment (start 187.29725 127.689686) (end 186.476564 126.869) (width 0.2) (layer "F.Cu") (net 15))
 (segment (start 160.49625 130.81) (end 166.287564 130.81) (width 0.2) (layer "F.Cu") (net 15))
 (segment (start 184.49525 128.850314) (end 185.315936 129.671) (width 0.2) (layer "F.Cu") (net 15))
 (segment (start 186.476564 110.621) (end 187.46975 109.627814) (width 0.2) (layer "F.Cu") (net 15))
 (segment (start 187.46975 90.6365) (end 185.26775 90.6365) (width 0.2) (layer "F.Cu") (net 15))
 (segment (start 185.26775 90.6365) (end 185.26775 88.927874) (width 0.2) (layer "F.Cu") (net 15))
 (segment (start 181.01094 87.202) (end 180.38825 87.82469) (width 0.2) (layer "F.Cu") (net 15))
 (segment (start 180.38825 87.82469) (end 180.38825 94.822) (width 0.2) (layer "F.Cu") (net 15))
 (segment (start 183.80325 99.226626) (end 183.80325 94.61937) (width 0.2) (layer "F.Cu") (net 5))
 (segment (start 181.01094 99.488) (end 183.541876 99.488) (width 0.2) (layer "F.Cu") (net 5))
 (segment (start 188.76775 90.3385) (end 190.96975 90.3385) (width 0.2) (layer "F.Cu") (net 5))
 (segment (start 168.31094 86.788) (end 181.01094 99.488) (width 0.2) (layer "F.Cu") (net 5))
 (segment (start 179.54625 130.81) (end 186.471764 130.81) (width 0.2) (layer "F.Cu") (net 5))
 (segment (start 186.18225 84.099) (end 162.3339 84.099) (width 0.2) (layer "F.Cu") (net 5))
 (segment (start 162.39475 90.3385) (end 162.39475 88.513874) (width 0.2) (layer "F.Cu") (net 5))
 (segment (start 183.80325 94.61937) (end 182.52888 93.345) (width 0.2) (layer "F.Cu") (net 5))
 (segment (start 164.120624 86.788) (end 168.31094 86.788) (width 0.2) (layer "F.Cu") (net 5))
 (segment (start 190.96975 90.3385) (end 190.96975 88.8865) (width 0.2) (layer "F.Cu") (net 5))
 (segment (start 160.19275 86.24015) (end 160.19275 90.3385) (width 0.2) (layer "F.Cu") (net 5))
 (segment (start 182.52888 93.345) (end 181.45125 93.345) (width 0.2) (layer "F.Cu") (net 5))
 (segment (start 183.541876 99.488) (end 183.80325 99.226626) (width 0.2) (layer "F.Cu") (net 5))
 (segment (start 190.96975 88.8865) (end 186.18225 84.099) (width 0.2) (layer "F.Cu") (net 5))
 (segment (start 189.63725 127.644514) (end 189.63725 97.1155) (width 0.2) (layer "F.Cu") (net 5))
 (segment (start 188.76775 96.246) (end 188.76775 90.3385) (width 0.2) (layer "F.Cu") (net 5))
 (segment (start 162.3339 84.099) (end 160.19275 86.24015) (width 0.2) (layer "F.Cu") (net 5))
 (segment (start 189.63725 97.1155) (end 188.76775 96.246) (width 0.2) (layer "F.Cu") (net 5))
 (segment (start 160.19275 90.3385) (end 162.39475 90.3385) (width 0.2) (layer "F.Cu") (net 5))
 (segment (start 162.39475 88.513874) (end 164.120624 86.788) (width 0.2) (layer "F.Cu") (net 5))
 (segment (start 186.471764 130.81) (end 189.63725 127.644514) (width 0.2) (layer "F.Cu") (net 5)))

